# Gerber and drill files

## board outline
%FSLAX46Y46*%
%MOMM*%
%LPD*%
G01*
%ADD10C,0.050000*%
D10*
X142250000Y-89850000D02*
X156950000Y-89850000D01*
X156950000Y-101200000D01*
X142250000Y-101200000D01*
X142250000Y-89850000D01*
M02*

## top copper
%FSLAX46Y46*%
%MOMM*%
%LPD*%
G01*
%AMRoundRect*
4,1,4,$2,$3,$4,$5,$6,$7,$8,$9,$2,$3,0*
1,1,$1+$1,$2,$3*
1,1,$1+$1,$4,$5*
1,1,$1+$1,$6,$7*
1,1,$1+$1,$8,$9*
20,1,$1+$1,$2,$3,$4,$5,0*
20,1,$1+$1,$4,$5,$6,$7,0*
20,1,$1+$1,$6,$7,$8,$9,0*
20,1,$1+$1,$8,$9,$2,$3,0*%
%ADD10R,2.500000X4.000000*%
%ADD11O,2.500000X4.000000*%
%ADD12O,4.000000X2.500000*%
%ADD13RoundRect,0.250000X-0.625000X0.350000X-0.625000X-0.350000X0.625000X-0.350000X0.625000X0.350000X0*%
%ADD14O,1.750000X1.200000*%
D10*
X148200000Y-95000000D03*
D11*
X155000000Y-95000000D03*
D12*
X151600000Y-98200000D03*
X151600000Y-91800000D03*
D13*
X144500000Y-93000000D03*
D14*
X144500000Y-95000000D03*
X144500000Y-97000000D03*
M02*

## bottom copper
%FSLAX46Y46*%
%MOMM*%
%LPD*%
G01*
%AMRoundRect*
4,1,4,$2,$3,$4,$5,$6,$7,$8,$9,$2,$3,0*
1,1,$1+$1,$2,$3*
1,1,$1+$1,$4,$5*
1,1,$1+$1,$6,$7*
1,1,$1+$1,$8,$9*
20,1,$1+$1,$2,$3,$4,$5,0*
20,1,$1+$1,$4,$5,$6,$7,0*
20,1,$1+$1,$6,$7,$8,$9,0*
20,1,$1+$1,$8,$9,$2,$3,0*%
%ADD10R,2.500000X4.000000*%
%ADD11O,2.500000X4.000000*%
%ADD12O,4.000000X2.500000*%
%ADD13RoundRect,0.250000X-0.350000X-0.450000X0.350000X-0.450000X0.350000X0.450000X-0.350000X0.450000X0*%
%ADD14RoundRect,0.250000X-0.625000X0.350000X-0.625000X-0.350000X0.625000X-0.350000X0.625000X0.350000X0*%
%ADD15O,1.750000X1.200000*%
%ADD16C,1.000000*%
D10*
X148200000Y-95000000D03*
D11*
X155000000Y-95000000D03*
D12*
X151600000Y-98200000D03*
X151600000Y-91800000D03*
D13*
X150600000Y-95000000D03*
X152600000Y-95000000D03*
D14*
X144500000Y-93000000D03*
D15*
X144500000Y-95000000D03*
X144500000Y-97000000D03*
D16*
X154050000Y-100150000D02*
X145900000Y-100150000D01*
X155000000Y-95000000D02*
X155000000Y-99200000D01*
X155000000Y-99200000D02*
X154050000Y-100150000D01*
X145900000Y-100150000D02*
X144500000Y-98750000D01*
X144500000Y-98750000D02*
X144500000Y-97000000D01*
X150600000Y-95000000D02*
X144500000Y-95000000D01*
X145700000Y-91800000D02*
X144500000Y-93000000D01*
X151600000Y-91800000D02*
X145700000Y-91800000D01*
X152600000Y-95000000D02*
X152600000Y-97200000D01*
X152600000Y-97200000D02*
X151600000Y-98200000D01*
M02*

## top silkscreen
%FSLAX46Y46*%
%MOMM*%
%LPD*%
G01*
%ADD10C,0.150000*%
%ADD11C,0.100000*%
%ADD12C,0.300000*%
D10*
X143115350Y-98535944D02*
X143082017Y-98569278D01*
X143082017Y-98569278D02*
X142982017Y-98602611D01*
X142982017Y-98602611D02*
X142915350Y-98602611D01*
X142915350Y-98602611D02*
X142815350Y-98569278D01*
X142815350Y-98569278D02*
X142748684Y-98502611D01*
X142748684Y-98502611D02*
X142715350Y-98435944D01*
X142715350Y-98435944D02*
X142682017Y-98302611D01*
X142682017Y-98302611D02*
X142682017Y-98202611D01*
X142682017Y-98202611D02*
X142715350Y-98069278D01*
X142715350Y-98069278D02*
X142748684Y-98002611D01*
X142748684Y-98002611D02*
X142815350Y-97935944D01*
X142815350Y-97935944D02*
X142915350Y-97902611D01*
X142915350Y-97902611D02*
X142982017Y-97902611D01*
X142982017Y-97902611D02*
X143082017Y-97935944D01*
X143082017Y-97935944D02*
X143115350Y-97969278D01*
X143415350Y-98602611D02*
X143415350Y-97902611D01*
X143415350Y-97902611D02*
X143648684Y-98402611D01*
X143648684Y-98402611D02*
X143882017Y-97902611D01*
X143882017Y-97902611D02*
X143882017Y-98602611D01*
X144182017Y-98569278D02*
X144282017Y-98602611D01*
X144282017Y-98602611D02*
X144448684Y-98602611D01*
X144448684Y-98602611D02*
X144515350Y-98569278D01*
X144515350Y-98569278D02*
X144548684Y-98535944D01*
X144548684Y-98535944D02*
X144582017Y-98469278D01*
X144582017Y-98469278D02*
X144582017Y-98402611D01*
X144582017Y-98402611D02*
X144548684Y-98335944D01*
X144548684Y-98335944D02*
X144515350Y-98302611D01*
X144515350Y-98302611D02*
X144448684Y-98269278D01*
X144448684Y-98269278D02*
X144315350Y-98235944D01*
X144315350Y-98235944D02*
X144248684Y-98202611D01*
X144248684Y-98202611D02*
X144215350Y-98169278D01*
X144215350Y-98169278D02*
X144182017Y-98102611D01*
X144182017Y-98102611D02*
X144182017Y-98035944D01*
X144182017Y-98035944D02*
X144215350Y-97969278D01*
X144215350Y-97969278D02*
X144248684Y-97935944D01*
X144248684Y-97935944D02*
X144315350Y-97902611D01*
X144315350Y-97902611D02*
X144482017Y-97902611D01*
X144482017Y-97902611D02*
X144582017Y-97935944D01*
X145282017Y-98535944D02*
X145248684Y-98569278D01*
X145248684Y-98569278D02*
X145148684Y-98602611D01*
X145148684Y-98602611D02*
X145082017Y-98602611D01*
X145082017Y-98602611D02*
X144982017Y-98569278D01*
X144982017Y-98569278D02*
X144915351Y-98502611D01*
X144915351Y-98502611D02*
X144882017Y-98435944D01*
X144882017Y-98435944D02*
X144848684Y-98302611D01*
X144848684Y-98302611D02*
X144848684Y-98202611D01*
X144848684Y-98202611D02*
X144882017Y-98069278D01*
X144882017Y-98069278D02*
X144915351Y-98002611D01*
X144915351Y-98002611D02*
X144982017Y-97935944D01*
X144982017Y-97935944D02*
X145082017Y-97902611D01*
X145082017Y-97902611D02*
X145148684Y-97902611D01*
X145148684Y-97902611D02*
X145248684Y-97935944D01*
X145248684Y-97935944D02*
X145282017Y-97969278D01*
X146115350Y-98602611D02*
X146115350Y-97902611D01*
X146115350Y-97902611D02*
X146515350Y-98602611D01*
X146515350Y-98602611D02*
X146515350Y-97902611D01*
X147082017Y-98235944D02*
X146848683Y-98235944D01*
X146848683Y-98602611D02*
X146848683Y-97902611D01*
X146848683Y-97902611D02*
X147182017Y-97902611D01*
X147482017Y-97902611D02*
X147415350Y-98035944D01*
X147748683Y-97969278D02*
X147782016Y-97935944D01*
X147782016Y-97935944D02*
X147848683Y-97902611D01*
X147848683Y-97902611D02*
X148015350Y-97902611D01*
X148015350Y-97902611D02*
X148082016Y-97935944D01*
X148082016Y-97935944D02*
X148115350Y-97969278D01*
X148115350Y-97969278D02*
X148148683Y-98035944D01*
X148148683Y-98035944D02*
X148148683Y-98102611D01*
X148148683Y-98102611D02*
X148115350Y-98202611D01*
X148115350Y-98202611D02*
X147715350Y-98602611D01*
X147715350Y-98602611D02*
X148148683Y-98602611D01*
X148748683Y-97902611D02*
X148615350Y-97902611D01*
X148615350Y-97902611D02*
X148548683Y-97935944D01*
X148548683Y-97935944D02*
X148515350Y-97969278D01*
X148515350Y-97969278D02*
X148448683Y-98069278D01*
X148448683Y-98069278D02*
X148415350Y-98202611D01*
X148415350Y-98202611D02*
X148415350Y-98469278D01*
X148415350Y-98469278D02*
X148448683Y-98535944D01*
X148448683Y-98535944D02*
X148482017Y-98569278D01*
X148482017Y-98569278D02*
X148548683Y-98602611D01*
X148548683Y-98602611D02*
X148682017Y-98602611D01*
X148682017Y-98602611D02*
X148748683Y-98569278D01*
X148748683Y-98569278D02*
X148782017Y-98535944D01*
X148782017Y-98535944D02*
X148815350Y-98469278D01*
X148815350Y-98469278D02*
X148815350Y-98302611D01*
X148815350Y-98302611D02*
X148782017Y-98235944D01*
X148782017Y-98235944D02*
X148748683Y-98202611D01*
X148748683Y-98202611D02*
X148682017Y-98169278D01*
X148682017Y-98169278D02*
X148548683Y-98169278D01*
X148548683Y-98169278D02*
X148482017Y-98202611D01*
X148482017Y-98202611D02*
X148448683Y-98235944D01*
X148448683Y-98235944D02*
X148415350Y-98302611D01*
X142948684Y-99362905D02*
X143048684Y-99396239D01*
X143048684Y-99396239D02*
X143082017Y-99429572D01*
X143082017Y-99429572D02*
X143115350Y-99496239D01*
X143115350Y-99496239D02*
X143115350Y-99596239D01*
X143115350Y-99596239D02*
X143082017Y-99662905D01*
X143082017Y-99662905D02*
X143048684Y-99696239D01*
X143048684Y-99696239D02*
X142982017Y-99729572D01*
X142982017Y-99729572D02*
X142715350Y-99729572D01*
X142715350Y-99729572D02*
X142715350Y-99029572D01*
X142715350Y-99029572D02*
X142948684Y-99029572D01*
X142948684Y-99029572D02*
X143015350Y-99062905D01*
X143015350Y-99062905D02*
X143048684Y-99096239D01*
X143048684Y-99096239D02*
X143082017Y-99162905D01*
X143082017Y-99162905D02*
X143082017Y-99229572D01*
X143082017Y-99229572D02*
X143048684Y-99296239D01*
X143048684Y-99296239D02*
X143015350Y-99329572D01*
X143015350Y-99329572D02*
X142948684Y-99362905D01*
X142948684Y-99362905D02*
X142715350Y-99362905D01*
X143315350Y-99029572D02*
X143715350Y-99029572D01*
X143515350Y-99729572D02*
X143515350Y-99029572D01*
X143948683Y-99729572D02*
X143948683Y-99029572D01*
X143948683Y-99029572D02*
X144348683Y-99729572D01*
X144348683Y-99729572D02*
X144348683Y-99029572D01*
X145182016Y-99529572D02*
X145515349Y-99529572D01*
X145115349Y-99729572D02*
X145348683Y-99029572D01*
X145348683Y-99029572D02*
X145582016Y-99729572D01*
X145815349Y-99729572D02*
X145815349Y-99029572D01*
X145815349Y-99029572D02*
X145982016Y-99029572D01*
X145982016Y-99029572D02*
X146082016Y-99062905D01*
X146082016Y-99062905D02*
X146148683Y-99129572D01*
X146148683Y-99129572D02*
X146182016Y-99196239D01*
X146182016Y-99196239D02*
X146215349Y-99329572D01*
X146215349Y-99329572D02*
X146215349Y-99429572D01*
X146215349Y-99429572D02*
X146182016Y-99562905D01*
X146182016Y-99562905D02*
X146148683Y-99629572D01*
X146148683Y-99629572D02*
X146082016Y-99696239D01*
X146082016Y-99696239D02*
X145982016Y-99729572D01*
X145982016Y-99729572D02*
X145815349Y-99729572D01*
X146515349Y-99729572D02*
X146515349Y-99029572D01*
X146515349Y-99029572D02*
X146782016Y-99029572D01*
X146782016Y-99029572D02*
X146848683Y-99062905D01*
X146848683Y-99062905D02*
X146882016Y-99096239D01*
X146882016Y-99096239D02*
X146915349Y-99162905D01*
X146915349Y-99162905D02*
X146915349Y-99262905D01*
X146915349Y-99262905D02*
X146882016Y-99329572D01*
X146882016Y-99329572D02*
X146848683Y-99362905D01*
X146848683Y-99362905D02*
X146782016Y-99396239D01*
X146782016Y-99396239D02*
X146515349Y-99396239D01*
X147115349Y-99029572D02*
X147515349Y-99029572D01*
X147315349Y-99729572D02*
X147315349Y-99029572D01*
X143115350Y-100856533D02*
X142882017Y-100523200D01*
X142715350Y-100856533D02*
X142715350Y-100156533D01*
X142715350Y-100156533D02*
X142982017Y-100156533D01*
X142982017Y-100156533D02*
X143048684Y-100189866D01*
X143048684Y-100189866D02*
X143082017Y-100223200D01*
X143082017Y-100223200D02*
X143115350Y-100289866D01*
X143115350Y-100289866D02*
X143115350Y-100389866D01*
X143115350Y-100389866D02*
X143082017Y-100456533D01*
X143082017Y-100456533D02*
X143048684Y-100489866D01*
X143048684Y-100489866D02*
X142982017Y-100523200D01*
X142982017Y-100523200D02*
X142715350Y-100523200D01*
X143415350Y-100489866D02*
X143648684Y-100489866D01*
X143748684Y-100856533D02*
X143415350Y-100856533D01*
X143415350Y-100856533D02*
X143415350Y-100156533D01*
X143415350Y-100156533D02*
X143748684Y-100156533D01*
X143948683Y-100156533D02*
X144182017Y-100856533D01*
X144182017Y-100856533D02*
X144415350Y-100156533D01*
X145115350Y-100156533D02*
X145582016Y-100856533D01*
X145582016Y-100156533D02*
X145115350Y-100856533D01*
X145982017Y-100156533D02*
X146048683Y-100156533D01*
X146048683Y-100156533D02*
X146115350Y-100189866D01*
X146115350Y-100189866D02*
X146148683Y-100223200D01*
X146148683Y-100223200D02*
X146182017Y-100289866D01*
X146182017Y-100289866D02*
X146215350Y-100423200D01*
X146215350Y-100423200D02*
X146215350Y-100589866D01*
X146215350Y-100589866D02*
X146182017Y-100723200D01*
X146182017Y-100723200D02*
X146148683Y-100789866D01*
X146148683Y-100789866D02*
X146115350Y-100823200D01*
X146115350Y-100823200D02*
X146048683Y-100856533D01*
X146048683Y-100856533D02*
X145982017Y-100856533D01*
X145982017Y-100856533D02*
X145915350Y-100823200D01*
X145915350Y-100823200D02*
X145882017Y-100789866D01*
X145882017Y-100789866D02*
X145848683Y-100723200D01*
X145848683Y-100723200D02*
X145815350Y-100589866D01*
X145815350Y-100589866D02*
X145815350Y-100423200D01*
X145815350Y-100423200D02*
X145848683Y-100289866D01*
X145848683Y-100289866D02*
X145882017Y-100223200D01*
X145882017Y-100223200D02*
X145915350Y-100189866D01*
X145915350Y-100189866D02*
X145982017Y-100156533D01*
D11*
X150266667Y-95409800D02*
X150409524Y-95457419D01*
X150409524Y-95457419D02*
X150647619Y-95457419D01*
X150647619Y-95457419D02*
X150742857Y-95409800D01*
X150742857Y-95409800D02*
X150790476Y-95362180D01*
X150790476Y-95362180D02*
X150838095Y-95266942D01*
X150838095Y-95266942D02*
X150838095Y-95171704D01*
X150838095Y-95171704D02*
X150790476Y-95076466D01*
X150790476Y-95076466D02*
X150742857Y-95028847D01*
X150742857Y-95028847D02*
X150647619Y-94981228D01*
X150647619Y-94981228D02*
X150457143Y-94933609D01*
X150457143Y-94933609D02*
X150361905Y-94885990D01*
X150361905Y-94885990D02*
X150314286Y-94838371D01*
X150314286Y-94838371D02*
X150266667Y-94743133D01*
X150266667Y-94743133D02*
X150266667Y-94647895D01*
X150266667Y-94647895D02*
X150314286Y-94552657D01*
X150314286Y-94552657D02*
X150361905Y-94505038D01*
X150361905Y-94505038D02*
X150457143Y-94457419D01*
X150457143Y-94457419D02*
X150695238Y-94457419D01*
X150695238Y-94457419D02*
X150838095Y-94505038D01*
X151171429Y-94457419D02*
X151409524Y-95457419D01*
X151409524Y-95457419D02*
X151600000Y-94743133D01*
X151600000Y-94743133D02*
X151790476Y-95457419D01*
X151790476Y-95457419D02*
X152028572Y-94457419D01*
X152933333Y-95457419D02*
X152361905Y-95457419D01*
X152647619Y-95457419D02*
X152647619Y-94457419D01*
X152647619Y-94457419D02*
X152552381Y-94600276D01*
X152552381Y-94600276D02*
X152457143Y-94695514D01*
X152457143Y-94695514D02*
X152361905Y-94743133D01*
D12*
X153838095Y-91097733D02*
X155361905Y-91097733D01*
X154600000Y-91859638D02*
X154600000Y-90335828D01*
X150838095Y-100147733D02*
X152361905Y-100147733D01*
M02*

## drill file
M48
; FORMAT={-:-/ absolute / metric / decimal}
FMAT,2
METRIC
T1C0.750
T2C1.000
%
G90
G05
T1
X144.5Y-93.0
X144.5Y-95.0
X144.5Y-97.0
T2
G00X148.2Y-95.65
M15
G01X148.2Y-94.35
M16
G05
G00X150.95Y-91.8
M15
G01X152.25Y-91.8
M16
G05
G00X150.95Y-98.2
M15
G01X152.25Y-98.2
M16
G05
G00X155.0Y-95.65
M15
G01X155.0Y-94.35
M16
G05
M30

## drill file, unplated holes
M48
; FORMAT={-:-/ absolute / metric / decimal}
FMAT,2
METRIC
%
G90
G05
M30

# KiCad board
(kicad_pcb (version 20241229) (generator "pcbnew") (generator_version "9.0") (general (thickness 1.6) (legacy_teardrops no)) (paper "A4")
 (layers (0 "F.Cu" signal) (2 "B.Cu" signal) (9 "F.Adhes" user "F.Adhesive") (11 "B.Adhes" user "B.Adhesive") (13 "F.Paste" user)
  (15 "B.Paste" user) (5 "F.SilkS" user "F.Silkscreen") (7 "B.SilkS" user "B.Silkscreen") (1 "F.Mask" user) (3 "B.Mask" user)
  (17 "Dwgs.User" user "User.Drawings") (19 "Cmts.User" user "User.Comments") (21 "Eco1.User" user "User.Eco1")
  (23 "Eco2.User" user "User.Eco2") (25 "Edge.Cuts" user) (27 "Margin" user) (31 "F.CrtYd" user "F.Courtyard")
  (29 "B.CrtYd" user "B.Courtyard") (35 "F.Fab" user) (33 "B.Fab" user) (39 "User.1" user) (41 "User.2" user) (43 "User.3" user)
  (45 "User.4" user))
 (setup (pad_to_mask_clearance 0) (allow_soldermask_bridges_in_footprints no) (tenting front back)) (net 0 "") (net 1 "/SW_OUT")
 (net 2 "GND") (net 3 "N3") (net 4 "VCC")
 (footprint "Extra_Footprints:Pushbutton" (layer "F.Cu") (at 151.6 95)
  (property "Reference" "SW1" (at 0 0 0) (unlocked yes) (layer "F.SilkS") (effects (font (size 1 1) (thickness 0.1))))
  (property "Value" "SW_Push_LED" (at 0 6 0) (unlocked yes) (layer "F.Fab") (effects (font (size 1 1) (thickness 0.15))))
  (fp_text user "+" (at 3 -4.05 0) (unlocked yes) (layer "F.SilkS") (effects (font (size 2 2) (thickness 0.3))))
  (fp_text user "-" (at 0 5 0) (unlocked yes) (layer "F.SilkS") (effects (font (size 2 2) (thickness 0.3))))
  (pad "1" thru_hole rect (at -3.4 0 90) (size 4 2.5) (drill oval 2.3 1) (layers "*.Cu" "*.Mask") (remove_unused_layers no)
   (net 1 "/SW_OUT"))
  (pad "2" thru_hole oval (at 3.4 0 90) (size 4 2.5) (drill oval 2.3 1) (layers "*.Cu" "*.Mask") (remove_unused_layers no) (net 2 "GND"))
  (pad "3" thru_hole oval (at 0 3.2) (size 4 2.5) (drill oval 2.3 1) (layers "*.Cu" "*.Mask") (remove_unused_layers no) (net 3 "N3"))
  (pad "4" thru_hole oval (at 0 -3.2) (size 4 2.5) (drill oval 2.3 1) (layers "*.Cu" "*.Mask") (remove_unused_layers no) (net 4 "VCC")))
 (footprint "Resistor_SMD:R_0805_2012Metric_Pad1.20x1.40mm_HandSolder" (layer "B.Cu") (at 151.6 95)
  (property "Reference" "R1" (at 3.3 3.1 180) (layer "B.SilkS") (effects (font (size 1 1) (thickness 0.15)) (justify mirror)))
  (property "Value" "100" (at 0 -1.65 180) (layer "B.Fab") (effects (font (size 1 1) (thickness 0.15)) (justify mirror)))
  (pad "1" smd roundrect (at -1 0) (size 1.2 1.4) (layers "B.Cu" "B.Mask" "B.Paste") (roundrect_rratio 0.208333) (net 1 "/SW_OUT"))
  (pad "2" smd roundrect (at 1 0) (size 1.2 1.4) (layers "B.Cu" "B.Mask" "B.Paste") (roundrect_rratio 0.208333) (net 3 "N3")))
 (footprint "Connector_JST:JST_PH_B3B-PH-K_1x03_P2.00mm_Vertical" (layer "B.Cu") (at 144.5 93 -90)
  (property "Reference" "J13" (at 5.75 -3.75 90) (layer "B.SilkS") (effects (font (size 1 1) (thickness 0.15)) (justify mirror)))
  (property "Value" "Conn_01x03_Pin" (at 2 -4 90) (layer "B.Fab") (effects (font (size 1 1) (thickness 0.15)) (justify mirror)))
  (pad "1" thru_hole roundrect (at 0 0 270) (size 1.2 1.75) (drill 0.75) (layers "*.Cu" "*.Mask") (remove_unused_layers no)
   (roundrect_rratio 0.208333) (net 4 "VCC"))
  (pad "2" thru_hole oval (at 2 0 270) (size 1.2 1.75) (drill 0.75) (layers "*.Cu" "*.Mask") (remove_unused_layers no) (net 1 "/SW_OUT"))
  (pad "3" thru_hole oval (at 4 0 270) (size 1.2 1.75) (drill 0.75) (layers "*.Cu" "*.Mask") (remove_unused_layers no) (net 2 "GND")))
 (gr_rect (start 142.25 89.85) (end 156.95 101.2) (stroke (width 0.05) (type default)) (fill no) (layer "Edge.Cuts"))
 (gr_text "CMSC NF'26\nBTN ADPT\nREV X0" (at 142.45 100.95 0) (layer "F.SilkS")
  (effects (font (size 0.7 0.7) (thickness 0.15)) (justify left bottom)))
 (segment (start 154.05 100.15) (end 145.9 100.15) (width 1) (layer "B.Cu") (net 2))
 (segment (start 155 95) (end 155 99.2) (width 1) (layer "B.Cu") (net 2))
 (segment (start 155 99.2) (end 154.05 100.15) (width 1) (layer "B.Cu") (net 2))
 (segment (start 145.9 100.15) (end 144.5 98.75) (width 1) (layer "B.Cu") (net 2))
 (segment (start 144.5 98.75) (end 144.5 97) (width 1) (layer "B.Cu") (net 2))
 (segment (start 150.6 95) (end 144.5 95) (width 1) (layer "B.Cu") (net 1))
 (segment (start 145.7 91.8) (end 144.5 93) (width 1) (layer "B.Cu") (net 4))
 (segment (start 151.6 91.8) (end 145.7 91.8) (width 1) (layer "B.Cu") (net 4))
 (segment (start 152.6 95) (end 152.6 97.2) (width 1) (layer "B.Cu") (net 3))
 (segment (start 152.6 97.2) (end 151.6 98.2) (width 1) (layer "B.Cu") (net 3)))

